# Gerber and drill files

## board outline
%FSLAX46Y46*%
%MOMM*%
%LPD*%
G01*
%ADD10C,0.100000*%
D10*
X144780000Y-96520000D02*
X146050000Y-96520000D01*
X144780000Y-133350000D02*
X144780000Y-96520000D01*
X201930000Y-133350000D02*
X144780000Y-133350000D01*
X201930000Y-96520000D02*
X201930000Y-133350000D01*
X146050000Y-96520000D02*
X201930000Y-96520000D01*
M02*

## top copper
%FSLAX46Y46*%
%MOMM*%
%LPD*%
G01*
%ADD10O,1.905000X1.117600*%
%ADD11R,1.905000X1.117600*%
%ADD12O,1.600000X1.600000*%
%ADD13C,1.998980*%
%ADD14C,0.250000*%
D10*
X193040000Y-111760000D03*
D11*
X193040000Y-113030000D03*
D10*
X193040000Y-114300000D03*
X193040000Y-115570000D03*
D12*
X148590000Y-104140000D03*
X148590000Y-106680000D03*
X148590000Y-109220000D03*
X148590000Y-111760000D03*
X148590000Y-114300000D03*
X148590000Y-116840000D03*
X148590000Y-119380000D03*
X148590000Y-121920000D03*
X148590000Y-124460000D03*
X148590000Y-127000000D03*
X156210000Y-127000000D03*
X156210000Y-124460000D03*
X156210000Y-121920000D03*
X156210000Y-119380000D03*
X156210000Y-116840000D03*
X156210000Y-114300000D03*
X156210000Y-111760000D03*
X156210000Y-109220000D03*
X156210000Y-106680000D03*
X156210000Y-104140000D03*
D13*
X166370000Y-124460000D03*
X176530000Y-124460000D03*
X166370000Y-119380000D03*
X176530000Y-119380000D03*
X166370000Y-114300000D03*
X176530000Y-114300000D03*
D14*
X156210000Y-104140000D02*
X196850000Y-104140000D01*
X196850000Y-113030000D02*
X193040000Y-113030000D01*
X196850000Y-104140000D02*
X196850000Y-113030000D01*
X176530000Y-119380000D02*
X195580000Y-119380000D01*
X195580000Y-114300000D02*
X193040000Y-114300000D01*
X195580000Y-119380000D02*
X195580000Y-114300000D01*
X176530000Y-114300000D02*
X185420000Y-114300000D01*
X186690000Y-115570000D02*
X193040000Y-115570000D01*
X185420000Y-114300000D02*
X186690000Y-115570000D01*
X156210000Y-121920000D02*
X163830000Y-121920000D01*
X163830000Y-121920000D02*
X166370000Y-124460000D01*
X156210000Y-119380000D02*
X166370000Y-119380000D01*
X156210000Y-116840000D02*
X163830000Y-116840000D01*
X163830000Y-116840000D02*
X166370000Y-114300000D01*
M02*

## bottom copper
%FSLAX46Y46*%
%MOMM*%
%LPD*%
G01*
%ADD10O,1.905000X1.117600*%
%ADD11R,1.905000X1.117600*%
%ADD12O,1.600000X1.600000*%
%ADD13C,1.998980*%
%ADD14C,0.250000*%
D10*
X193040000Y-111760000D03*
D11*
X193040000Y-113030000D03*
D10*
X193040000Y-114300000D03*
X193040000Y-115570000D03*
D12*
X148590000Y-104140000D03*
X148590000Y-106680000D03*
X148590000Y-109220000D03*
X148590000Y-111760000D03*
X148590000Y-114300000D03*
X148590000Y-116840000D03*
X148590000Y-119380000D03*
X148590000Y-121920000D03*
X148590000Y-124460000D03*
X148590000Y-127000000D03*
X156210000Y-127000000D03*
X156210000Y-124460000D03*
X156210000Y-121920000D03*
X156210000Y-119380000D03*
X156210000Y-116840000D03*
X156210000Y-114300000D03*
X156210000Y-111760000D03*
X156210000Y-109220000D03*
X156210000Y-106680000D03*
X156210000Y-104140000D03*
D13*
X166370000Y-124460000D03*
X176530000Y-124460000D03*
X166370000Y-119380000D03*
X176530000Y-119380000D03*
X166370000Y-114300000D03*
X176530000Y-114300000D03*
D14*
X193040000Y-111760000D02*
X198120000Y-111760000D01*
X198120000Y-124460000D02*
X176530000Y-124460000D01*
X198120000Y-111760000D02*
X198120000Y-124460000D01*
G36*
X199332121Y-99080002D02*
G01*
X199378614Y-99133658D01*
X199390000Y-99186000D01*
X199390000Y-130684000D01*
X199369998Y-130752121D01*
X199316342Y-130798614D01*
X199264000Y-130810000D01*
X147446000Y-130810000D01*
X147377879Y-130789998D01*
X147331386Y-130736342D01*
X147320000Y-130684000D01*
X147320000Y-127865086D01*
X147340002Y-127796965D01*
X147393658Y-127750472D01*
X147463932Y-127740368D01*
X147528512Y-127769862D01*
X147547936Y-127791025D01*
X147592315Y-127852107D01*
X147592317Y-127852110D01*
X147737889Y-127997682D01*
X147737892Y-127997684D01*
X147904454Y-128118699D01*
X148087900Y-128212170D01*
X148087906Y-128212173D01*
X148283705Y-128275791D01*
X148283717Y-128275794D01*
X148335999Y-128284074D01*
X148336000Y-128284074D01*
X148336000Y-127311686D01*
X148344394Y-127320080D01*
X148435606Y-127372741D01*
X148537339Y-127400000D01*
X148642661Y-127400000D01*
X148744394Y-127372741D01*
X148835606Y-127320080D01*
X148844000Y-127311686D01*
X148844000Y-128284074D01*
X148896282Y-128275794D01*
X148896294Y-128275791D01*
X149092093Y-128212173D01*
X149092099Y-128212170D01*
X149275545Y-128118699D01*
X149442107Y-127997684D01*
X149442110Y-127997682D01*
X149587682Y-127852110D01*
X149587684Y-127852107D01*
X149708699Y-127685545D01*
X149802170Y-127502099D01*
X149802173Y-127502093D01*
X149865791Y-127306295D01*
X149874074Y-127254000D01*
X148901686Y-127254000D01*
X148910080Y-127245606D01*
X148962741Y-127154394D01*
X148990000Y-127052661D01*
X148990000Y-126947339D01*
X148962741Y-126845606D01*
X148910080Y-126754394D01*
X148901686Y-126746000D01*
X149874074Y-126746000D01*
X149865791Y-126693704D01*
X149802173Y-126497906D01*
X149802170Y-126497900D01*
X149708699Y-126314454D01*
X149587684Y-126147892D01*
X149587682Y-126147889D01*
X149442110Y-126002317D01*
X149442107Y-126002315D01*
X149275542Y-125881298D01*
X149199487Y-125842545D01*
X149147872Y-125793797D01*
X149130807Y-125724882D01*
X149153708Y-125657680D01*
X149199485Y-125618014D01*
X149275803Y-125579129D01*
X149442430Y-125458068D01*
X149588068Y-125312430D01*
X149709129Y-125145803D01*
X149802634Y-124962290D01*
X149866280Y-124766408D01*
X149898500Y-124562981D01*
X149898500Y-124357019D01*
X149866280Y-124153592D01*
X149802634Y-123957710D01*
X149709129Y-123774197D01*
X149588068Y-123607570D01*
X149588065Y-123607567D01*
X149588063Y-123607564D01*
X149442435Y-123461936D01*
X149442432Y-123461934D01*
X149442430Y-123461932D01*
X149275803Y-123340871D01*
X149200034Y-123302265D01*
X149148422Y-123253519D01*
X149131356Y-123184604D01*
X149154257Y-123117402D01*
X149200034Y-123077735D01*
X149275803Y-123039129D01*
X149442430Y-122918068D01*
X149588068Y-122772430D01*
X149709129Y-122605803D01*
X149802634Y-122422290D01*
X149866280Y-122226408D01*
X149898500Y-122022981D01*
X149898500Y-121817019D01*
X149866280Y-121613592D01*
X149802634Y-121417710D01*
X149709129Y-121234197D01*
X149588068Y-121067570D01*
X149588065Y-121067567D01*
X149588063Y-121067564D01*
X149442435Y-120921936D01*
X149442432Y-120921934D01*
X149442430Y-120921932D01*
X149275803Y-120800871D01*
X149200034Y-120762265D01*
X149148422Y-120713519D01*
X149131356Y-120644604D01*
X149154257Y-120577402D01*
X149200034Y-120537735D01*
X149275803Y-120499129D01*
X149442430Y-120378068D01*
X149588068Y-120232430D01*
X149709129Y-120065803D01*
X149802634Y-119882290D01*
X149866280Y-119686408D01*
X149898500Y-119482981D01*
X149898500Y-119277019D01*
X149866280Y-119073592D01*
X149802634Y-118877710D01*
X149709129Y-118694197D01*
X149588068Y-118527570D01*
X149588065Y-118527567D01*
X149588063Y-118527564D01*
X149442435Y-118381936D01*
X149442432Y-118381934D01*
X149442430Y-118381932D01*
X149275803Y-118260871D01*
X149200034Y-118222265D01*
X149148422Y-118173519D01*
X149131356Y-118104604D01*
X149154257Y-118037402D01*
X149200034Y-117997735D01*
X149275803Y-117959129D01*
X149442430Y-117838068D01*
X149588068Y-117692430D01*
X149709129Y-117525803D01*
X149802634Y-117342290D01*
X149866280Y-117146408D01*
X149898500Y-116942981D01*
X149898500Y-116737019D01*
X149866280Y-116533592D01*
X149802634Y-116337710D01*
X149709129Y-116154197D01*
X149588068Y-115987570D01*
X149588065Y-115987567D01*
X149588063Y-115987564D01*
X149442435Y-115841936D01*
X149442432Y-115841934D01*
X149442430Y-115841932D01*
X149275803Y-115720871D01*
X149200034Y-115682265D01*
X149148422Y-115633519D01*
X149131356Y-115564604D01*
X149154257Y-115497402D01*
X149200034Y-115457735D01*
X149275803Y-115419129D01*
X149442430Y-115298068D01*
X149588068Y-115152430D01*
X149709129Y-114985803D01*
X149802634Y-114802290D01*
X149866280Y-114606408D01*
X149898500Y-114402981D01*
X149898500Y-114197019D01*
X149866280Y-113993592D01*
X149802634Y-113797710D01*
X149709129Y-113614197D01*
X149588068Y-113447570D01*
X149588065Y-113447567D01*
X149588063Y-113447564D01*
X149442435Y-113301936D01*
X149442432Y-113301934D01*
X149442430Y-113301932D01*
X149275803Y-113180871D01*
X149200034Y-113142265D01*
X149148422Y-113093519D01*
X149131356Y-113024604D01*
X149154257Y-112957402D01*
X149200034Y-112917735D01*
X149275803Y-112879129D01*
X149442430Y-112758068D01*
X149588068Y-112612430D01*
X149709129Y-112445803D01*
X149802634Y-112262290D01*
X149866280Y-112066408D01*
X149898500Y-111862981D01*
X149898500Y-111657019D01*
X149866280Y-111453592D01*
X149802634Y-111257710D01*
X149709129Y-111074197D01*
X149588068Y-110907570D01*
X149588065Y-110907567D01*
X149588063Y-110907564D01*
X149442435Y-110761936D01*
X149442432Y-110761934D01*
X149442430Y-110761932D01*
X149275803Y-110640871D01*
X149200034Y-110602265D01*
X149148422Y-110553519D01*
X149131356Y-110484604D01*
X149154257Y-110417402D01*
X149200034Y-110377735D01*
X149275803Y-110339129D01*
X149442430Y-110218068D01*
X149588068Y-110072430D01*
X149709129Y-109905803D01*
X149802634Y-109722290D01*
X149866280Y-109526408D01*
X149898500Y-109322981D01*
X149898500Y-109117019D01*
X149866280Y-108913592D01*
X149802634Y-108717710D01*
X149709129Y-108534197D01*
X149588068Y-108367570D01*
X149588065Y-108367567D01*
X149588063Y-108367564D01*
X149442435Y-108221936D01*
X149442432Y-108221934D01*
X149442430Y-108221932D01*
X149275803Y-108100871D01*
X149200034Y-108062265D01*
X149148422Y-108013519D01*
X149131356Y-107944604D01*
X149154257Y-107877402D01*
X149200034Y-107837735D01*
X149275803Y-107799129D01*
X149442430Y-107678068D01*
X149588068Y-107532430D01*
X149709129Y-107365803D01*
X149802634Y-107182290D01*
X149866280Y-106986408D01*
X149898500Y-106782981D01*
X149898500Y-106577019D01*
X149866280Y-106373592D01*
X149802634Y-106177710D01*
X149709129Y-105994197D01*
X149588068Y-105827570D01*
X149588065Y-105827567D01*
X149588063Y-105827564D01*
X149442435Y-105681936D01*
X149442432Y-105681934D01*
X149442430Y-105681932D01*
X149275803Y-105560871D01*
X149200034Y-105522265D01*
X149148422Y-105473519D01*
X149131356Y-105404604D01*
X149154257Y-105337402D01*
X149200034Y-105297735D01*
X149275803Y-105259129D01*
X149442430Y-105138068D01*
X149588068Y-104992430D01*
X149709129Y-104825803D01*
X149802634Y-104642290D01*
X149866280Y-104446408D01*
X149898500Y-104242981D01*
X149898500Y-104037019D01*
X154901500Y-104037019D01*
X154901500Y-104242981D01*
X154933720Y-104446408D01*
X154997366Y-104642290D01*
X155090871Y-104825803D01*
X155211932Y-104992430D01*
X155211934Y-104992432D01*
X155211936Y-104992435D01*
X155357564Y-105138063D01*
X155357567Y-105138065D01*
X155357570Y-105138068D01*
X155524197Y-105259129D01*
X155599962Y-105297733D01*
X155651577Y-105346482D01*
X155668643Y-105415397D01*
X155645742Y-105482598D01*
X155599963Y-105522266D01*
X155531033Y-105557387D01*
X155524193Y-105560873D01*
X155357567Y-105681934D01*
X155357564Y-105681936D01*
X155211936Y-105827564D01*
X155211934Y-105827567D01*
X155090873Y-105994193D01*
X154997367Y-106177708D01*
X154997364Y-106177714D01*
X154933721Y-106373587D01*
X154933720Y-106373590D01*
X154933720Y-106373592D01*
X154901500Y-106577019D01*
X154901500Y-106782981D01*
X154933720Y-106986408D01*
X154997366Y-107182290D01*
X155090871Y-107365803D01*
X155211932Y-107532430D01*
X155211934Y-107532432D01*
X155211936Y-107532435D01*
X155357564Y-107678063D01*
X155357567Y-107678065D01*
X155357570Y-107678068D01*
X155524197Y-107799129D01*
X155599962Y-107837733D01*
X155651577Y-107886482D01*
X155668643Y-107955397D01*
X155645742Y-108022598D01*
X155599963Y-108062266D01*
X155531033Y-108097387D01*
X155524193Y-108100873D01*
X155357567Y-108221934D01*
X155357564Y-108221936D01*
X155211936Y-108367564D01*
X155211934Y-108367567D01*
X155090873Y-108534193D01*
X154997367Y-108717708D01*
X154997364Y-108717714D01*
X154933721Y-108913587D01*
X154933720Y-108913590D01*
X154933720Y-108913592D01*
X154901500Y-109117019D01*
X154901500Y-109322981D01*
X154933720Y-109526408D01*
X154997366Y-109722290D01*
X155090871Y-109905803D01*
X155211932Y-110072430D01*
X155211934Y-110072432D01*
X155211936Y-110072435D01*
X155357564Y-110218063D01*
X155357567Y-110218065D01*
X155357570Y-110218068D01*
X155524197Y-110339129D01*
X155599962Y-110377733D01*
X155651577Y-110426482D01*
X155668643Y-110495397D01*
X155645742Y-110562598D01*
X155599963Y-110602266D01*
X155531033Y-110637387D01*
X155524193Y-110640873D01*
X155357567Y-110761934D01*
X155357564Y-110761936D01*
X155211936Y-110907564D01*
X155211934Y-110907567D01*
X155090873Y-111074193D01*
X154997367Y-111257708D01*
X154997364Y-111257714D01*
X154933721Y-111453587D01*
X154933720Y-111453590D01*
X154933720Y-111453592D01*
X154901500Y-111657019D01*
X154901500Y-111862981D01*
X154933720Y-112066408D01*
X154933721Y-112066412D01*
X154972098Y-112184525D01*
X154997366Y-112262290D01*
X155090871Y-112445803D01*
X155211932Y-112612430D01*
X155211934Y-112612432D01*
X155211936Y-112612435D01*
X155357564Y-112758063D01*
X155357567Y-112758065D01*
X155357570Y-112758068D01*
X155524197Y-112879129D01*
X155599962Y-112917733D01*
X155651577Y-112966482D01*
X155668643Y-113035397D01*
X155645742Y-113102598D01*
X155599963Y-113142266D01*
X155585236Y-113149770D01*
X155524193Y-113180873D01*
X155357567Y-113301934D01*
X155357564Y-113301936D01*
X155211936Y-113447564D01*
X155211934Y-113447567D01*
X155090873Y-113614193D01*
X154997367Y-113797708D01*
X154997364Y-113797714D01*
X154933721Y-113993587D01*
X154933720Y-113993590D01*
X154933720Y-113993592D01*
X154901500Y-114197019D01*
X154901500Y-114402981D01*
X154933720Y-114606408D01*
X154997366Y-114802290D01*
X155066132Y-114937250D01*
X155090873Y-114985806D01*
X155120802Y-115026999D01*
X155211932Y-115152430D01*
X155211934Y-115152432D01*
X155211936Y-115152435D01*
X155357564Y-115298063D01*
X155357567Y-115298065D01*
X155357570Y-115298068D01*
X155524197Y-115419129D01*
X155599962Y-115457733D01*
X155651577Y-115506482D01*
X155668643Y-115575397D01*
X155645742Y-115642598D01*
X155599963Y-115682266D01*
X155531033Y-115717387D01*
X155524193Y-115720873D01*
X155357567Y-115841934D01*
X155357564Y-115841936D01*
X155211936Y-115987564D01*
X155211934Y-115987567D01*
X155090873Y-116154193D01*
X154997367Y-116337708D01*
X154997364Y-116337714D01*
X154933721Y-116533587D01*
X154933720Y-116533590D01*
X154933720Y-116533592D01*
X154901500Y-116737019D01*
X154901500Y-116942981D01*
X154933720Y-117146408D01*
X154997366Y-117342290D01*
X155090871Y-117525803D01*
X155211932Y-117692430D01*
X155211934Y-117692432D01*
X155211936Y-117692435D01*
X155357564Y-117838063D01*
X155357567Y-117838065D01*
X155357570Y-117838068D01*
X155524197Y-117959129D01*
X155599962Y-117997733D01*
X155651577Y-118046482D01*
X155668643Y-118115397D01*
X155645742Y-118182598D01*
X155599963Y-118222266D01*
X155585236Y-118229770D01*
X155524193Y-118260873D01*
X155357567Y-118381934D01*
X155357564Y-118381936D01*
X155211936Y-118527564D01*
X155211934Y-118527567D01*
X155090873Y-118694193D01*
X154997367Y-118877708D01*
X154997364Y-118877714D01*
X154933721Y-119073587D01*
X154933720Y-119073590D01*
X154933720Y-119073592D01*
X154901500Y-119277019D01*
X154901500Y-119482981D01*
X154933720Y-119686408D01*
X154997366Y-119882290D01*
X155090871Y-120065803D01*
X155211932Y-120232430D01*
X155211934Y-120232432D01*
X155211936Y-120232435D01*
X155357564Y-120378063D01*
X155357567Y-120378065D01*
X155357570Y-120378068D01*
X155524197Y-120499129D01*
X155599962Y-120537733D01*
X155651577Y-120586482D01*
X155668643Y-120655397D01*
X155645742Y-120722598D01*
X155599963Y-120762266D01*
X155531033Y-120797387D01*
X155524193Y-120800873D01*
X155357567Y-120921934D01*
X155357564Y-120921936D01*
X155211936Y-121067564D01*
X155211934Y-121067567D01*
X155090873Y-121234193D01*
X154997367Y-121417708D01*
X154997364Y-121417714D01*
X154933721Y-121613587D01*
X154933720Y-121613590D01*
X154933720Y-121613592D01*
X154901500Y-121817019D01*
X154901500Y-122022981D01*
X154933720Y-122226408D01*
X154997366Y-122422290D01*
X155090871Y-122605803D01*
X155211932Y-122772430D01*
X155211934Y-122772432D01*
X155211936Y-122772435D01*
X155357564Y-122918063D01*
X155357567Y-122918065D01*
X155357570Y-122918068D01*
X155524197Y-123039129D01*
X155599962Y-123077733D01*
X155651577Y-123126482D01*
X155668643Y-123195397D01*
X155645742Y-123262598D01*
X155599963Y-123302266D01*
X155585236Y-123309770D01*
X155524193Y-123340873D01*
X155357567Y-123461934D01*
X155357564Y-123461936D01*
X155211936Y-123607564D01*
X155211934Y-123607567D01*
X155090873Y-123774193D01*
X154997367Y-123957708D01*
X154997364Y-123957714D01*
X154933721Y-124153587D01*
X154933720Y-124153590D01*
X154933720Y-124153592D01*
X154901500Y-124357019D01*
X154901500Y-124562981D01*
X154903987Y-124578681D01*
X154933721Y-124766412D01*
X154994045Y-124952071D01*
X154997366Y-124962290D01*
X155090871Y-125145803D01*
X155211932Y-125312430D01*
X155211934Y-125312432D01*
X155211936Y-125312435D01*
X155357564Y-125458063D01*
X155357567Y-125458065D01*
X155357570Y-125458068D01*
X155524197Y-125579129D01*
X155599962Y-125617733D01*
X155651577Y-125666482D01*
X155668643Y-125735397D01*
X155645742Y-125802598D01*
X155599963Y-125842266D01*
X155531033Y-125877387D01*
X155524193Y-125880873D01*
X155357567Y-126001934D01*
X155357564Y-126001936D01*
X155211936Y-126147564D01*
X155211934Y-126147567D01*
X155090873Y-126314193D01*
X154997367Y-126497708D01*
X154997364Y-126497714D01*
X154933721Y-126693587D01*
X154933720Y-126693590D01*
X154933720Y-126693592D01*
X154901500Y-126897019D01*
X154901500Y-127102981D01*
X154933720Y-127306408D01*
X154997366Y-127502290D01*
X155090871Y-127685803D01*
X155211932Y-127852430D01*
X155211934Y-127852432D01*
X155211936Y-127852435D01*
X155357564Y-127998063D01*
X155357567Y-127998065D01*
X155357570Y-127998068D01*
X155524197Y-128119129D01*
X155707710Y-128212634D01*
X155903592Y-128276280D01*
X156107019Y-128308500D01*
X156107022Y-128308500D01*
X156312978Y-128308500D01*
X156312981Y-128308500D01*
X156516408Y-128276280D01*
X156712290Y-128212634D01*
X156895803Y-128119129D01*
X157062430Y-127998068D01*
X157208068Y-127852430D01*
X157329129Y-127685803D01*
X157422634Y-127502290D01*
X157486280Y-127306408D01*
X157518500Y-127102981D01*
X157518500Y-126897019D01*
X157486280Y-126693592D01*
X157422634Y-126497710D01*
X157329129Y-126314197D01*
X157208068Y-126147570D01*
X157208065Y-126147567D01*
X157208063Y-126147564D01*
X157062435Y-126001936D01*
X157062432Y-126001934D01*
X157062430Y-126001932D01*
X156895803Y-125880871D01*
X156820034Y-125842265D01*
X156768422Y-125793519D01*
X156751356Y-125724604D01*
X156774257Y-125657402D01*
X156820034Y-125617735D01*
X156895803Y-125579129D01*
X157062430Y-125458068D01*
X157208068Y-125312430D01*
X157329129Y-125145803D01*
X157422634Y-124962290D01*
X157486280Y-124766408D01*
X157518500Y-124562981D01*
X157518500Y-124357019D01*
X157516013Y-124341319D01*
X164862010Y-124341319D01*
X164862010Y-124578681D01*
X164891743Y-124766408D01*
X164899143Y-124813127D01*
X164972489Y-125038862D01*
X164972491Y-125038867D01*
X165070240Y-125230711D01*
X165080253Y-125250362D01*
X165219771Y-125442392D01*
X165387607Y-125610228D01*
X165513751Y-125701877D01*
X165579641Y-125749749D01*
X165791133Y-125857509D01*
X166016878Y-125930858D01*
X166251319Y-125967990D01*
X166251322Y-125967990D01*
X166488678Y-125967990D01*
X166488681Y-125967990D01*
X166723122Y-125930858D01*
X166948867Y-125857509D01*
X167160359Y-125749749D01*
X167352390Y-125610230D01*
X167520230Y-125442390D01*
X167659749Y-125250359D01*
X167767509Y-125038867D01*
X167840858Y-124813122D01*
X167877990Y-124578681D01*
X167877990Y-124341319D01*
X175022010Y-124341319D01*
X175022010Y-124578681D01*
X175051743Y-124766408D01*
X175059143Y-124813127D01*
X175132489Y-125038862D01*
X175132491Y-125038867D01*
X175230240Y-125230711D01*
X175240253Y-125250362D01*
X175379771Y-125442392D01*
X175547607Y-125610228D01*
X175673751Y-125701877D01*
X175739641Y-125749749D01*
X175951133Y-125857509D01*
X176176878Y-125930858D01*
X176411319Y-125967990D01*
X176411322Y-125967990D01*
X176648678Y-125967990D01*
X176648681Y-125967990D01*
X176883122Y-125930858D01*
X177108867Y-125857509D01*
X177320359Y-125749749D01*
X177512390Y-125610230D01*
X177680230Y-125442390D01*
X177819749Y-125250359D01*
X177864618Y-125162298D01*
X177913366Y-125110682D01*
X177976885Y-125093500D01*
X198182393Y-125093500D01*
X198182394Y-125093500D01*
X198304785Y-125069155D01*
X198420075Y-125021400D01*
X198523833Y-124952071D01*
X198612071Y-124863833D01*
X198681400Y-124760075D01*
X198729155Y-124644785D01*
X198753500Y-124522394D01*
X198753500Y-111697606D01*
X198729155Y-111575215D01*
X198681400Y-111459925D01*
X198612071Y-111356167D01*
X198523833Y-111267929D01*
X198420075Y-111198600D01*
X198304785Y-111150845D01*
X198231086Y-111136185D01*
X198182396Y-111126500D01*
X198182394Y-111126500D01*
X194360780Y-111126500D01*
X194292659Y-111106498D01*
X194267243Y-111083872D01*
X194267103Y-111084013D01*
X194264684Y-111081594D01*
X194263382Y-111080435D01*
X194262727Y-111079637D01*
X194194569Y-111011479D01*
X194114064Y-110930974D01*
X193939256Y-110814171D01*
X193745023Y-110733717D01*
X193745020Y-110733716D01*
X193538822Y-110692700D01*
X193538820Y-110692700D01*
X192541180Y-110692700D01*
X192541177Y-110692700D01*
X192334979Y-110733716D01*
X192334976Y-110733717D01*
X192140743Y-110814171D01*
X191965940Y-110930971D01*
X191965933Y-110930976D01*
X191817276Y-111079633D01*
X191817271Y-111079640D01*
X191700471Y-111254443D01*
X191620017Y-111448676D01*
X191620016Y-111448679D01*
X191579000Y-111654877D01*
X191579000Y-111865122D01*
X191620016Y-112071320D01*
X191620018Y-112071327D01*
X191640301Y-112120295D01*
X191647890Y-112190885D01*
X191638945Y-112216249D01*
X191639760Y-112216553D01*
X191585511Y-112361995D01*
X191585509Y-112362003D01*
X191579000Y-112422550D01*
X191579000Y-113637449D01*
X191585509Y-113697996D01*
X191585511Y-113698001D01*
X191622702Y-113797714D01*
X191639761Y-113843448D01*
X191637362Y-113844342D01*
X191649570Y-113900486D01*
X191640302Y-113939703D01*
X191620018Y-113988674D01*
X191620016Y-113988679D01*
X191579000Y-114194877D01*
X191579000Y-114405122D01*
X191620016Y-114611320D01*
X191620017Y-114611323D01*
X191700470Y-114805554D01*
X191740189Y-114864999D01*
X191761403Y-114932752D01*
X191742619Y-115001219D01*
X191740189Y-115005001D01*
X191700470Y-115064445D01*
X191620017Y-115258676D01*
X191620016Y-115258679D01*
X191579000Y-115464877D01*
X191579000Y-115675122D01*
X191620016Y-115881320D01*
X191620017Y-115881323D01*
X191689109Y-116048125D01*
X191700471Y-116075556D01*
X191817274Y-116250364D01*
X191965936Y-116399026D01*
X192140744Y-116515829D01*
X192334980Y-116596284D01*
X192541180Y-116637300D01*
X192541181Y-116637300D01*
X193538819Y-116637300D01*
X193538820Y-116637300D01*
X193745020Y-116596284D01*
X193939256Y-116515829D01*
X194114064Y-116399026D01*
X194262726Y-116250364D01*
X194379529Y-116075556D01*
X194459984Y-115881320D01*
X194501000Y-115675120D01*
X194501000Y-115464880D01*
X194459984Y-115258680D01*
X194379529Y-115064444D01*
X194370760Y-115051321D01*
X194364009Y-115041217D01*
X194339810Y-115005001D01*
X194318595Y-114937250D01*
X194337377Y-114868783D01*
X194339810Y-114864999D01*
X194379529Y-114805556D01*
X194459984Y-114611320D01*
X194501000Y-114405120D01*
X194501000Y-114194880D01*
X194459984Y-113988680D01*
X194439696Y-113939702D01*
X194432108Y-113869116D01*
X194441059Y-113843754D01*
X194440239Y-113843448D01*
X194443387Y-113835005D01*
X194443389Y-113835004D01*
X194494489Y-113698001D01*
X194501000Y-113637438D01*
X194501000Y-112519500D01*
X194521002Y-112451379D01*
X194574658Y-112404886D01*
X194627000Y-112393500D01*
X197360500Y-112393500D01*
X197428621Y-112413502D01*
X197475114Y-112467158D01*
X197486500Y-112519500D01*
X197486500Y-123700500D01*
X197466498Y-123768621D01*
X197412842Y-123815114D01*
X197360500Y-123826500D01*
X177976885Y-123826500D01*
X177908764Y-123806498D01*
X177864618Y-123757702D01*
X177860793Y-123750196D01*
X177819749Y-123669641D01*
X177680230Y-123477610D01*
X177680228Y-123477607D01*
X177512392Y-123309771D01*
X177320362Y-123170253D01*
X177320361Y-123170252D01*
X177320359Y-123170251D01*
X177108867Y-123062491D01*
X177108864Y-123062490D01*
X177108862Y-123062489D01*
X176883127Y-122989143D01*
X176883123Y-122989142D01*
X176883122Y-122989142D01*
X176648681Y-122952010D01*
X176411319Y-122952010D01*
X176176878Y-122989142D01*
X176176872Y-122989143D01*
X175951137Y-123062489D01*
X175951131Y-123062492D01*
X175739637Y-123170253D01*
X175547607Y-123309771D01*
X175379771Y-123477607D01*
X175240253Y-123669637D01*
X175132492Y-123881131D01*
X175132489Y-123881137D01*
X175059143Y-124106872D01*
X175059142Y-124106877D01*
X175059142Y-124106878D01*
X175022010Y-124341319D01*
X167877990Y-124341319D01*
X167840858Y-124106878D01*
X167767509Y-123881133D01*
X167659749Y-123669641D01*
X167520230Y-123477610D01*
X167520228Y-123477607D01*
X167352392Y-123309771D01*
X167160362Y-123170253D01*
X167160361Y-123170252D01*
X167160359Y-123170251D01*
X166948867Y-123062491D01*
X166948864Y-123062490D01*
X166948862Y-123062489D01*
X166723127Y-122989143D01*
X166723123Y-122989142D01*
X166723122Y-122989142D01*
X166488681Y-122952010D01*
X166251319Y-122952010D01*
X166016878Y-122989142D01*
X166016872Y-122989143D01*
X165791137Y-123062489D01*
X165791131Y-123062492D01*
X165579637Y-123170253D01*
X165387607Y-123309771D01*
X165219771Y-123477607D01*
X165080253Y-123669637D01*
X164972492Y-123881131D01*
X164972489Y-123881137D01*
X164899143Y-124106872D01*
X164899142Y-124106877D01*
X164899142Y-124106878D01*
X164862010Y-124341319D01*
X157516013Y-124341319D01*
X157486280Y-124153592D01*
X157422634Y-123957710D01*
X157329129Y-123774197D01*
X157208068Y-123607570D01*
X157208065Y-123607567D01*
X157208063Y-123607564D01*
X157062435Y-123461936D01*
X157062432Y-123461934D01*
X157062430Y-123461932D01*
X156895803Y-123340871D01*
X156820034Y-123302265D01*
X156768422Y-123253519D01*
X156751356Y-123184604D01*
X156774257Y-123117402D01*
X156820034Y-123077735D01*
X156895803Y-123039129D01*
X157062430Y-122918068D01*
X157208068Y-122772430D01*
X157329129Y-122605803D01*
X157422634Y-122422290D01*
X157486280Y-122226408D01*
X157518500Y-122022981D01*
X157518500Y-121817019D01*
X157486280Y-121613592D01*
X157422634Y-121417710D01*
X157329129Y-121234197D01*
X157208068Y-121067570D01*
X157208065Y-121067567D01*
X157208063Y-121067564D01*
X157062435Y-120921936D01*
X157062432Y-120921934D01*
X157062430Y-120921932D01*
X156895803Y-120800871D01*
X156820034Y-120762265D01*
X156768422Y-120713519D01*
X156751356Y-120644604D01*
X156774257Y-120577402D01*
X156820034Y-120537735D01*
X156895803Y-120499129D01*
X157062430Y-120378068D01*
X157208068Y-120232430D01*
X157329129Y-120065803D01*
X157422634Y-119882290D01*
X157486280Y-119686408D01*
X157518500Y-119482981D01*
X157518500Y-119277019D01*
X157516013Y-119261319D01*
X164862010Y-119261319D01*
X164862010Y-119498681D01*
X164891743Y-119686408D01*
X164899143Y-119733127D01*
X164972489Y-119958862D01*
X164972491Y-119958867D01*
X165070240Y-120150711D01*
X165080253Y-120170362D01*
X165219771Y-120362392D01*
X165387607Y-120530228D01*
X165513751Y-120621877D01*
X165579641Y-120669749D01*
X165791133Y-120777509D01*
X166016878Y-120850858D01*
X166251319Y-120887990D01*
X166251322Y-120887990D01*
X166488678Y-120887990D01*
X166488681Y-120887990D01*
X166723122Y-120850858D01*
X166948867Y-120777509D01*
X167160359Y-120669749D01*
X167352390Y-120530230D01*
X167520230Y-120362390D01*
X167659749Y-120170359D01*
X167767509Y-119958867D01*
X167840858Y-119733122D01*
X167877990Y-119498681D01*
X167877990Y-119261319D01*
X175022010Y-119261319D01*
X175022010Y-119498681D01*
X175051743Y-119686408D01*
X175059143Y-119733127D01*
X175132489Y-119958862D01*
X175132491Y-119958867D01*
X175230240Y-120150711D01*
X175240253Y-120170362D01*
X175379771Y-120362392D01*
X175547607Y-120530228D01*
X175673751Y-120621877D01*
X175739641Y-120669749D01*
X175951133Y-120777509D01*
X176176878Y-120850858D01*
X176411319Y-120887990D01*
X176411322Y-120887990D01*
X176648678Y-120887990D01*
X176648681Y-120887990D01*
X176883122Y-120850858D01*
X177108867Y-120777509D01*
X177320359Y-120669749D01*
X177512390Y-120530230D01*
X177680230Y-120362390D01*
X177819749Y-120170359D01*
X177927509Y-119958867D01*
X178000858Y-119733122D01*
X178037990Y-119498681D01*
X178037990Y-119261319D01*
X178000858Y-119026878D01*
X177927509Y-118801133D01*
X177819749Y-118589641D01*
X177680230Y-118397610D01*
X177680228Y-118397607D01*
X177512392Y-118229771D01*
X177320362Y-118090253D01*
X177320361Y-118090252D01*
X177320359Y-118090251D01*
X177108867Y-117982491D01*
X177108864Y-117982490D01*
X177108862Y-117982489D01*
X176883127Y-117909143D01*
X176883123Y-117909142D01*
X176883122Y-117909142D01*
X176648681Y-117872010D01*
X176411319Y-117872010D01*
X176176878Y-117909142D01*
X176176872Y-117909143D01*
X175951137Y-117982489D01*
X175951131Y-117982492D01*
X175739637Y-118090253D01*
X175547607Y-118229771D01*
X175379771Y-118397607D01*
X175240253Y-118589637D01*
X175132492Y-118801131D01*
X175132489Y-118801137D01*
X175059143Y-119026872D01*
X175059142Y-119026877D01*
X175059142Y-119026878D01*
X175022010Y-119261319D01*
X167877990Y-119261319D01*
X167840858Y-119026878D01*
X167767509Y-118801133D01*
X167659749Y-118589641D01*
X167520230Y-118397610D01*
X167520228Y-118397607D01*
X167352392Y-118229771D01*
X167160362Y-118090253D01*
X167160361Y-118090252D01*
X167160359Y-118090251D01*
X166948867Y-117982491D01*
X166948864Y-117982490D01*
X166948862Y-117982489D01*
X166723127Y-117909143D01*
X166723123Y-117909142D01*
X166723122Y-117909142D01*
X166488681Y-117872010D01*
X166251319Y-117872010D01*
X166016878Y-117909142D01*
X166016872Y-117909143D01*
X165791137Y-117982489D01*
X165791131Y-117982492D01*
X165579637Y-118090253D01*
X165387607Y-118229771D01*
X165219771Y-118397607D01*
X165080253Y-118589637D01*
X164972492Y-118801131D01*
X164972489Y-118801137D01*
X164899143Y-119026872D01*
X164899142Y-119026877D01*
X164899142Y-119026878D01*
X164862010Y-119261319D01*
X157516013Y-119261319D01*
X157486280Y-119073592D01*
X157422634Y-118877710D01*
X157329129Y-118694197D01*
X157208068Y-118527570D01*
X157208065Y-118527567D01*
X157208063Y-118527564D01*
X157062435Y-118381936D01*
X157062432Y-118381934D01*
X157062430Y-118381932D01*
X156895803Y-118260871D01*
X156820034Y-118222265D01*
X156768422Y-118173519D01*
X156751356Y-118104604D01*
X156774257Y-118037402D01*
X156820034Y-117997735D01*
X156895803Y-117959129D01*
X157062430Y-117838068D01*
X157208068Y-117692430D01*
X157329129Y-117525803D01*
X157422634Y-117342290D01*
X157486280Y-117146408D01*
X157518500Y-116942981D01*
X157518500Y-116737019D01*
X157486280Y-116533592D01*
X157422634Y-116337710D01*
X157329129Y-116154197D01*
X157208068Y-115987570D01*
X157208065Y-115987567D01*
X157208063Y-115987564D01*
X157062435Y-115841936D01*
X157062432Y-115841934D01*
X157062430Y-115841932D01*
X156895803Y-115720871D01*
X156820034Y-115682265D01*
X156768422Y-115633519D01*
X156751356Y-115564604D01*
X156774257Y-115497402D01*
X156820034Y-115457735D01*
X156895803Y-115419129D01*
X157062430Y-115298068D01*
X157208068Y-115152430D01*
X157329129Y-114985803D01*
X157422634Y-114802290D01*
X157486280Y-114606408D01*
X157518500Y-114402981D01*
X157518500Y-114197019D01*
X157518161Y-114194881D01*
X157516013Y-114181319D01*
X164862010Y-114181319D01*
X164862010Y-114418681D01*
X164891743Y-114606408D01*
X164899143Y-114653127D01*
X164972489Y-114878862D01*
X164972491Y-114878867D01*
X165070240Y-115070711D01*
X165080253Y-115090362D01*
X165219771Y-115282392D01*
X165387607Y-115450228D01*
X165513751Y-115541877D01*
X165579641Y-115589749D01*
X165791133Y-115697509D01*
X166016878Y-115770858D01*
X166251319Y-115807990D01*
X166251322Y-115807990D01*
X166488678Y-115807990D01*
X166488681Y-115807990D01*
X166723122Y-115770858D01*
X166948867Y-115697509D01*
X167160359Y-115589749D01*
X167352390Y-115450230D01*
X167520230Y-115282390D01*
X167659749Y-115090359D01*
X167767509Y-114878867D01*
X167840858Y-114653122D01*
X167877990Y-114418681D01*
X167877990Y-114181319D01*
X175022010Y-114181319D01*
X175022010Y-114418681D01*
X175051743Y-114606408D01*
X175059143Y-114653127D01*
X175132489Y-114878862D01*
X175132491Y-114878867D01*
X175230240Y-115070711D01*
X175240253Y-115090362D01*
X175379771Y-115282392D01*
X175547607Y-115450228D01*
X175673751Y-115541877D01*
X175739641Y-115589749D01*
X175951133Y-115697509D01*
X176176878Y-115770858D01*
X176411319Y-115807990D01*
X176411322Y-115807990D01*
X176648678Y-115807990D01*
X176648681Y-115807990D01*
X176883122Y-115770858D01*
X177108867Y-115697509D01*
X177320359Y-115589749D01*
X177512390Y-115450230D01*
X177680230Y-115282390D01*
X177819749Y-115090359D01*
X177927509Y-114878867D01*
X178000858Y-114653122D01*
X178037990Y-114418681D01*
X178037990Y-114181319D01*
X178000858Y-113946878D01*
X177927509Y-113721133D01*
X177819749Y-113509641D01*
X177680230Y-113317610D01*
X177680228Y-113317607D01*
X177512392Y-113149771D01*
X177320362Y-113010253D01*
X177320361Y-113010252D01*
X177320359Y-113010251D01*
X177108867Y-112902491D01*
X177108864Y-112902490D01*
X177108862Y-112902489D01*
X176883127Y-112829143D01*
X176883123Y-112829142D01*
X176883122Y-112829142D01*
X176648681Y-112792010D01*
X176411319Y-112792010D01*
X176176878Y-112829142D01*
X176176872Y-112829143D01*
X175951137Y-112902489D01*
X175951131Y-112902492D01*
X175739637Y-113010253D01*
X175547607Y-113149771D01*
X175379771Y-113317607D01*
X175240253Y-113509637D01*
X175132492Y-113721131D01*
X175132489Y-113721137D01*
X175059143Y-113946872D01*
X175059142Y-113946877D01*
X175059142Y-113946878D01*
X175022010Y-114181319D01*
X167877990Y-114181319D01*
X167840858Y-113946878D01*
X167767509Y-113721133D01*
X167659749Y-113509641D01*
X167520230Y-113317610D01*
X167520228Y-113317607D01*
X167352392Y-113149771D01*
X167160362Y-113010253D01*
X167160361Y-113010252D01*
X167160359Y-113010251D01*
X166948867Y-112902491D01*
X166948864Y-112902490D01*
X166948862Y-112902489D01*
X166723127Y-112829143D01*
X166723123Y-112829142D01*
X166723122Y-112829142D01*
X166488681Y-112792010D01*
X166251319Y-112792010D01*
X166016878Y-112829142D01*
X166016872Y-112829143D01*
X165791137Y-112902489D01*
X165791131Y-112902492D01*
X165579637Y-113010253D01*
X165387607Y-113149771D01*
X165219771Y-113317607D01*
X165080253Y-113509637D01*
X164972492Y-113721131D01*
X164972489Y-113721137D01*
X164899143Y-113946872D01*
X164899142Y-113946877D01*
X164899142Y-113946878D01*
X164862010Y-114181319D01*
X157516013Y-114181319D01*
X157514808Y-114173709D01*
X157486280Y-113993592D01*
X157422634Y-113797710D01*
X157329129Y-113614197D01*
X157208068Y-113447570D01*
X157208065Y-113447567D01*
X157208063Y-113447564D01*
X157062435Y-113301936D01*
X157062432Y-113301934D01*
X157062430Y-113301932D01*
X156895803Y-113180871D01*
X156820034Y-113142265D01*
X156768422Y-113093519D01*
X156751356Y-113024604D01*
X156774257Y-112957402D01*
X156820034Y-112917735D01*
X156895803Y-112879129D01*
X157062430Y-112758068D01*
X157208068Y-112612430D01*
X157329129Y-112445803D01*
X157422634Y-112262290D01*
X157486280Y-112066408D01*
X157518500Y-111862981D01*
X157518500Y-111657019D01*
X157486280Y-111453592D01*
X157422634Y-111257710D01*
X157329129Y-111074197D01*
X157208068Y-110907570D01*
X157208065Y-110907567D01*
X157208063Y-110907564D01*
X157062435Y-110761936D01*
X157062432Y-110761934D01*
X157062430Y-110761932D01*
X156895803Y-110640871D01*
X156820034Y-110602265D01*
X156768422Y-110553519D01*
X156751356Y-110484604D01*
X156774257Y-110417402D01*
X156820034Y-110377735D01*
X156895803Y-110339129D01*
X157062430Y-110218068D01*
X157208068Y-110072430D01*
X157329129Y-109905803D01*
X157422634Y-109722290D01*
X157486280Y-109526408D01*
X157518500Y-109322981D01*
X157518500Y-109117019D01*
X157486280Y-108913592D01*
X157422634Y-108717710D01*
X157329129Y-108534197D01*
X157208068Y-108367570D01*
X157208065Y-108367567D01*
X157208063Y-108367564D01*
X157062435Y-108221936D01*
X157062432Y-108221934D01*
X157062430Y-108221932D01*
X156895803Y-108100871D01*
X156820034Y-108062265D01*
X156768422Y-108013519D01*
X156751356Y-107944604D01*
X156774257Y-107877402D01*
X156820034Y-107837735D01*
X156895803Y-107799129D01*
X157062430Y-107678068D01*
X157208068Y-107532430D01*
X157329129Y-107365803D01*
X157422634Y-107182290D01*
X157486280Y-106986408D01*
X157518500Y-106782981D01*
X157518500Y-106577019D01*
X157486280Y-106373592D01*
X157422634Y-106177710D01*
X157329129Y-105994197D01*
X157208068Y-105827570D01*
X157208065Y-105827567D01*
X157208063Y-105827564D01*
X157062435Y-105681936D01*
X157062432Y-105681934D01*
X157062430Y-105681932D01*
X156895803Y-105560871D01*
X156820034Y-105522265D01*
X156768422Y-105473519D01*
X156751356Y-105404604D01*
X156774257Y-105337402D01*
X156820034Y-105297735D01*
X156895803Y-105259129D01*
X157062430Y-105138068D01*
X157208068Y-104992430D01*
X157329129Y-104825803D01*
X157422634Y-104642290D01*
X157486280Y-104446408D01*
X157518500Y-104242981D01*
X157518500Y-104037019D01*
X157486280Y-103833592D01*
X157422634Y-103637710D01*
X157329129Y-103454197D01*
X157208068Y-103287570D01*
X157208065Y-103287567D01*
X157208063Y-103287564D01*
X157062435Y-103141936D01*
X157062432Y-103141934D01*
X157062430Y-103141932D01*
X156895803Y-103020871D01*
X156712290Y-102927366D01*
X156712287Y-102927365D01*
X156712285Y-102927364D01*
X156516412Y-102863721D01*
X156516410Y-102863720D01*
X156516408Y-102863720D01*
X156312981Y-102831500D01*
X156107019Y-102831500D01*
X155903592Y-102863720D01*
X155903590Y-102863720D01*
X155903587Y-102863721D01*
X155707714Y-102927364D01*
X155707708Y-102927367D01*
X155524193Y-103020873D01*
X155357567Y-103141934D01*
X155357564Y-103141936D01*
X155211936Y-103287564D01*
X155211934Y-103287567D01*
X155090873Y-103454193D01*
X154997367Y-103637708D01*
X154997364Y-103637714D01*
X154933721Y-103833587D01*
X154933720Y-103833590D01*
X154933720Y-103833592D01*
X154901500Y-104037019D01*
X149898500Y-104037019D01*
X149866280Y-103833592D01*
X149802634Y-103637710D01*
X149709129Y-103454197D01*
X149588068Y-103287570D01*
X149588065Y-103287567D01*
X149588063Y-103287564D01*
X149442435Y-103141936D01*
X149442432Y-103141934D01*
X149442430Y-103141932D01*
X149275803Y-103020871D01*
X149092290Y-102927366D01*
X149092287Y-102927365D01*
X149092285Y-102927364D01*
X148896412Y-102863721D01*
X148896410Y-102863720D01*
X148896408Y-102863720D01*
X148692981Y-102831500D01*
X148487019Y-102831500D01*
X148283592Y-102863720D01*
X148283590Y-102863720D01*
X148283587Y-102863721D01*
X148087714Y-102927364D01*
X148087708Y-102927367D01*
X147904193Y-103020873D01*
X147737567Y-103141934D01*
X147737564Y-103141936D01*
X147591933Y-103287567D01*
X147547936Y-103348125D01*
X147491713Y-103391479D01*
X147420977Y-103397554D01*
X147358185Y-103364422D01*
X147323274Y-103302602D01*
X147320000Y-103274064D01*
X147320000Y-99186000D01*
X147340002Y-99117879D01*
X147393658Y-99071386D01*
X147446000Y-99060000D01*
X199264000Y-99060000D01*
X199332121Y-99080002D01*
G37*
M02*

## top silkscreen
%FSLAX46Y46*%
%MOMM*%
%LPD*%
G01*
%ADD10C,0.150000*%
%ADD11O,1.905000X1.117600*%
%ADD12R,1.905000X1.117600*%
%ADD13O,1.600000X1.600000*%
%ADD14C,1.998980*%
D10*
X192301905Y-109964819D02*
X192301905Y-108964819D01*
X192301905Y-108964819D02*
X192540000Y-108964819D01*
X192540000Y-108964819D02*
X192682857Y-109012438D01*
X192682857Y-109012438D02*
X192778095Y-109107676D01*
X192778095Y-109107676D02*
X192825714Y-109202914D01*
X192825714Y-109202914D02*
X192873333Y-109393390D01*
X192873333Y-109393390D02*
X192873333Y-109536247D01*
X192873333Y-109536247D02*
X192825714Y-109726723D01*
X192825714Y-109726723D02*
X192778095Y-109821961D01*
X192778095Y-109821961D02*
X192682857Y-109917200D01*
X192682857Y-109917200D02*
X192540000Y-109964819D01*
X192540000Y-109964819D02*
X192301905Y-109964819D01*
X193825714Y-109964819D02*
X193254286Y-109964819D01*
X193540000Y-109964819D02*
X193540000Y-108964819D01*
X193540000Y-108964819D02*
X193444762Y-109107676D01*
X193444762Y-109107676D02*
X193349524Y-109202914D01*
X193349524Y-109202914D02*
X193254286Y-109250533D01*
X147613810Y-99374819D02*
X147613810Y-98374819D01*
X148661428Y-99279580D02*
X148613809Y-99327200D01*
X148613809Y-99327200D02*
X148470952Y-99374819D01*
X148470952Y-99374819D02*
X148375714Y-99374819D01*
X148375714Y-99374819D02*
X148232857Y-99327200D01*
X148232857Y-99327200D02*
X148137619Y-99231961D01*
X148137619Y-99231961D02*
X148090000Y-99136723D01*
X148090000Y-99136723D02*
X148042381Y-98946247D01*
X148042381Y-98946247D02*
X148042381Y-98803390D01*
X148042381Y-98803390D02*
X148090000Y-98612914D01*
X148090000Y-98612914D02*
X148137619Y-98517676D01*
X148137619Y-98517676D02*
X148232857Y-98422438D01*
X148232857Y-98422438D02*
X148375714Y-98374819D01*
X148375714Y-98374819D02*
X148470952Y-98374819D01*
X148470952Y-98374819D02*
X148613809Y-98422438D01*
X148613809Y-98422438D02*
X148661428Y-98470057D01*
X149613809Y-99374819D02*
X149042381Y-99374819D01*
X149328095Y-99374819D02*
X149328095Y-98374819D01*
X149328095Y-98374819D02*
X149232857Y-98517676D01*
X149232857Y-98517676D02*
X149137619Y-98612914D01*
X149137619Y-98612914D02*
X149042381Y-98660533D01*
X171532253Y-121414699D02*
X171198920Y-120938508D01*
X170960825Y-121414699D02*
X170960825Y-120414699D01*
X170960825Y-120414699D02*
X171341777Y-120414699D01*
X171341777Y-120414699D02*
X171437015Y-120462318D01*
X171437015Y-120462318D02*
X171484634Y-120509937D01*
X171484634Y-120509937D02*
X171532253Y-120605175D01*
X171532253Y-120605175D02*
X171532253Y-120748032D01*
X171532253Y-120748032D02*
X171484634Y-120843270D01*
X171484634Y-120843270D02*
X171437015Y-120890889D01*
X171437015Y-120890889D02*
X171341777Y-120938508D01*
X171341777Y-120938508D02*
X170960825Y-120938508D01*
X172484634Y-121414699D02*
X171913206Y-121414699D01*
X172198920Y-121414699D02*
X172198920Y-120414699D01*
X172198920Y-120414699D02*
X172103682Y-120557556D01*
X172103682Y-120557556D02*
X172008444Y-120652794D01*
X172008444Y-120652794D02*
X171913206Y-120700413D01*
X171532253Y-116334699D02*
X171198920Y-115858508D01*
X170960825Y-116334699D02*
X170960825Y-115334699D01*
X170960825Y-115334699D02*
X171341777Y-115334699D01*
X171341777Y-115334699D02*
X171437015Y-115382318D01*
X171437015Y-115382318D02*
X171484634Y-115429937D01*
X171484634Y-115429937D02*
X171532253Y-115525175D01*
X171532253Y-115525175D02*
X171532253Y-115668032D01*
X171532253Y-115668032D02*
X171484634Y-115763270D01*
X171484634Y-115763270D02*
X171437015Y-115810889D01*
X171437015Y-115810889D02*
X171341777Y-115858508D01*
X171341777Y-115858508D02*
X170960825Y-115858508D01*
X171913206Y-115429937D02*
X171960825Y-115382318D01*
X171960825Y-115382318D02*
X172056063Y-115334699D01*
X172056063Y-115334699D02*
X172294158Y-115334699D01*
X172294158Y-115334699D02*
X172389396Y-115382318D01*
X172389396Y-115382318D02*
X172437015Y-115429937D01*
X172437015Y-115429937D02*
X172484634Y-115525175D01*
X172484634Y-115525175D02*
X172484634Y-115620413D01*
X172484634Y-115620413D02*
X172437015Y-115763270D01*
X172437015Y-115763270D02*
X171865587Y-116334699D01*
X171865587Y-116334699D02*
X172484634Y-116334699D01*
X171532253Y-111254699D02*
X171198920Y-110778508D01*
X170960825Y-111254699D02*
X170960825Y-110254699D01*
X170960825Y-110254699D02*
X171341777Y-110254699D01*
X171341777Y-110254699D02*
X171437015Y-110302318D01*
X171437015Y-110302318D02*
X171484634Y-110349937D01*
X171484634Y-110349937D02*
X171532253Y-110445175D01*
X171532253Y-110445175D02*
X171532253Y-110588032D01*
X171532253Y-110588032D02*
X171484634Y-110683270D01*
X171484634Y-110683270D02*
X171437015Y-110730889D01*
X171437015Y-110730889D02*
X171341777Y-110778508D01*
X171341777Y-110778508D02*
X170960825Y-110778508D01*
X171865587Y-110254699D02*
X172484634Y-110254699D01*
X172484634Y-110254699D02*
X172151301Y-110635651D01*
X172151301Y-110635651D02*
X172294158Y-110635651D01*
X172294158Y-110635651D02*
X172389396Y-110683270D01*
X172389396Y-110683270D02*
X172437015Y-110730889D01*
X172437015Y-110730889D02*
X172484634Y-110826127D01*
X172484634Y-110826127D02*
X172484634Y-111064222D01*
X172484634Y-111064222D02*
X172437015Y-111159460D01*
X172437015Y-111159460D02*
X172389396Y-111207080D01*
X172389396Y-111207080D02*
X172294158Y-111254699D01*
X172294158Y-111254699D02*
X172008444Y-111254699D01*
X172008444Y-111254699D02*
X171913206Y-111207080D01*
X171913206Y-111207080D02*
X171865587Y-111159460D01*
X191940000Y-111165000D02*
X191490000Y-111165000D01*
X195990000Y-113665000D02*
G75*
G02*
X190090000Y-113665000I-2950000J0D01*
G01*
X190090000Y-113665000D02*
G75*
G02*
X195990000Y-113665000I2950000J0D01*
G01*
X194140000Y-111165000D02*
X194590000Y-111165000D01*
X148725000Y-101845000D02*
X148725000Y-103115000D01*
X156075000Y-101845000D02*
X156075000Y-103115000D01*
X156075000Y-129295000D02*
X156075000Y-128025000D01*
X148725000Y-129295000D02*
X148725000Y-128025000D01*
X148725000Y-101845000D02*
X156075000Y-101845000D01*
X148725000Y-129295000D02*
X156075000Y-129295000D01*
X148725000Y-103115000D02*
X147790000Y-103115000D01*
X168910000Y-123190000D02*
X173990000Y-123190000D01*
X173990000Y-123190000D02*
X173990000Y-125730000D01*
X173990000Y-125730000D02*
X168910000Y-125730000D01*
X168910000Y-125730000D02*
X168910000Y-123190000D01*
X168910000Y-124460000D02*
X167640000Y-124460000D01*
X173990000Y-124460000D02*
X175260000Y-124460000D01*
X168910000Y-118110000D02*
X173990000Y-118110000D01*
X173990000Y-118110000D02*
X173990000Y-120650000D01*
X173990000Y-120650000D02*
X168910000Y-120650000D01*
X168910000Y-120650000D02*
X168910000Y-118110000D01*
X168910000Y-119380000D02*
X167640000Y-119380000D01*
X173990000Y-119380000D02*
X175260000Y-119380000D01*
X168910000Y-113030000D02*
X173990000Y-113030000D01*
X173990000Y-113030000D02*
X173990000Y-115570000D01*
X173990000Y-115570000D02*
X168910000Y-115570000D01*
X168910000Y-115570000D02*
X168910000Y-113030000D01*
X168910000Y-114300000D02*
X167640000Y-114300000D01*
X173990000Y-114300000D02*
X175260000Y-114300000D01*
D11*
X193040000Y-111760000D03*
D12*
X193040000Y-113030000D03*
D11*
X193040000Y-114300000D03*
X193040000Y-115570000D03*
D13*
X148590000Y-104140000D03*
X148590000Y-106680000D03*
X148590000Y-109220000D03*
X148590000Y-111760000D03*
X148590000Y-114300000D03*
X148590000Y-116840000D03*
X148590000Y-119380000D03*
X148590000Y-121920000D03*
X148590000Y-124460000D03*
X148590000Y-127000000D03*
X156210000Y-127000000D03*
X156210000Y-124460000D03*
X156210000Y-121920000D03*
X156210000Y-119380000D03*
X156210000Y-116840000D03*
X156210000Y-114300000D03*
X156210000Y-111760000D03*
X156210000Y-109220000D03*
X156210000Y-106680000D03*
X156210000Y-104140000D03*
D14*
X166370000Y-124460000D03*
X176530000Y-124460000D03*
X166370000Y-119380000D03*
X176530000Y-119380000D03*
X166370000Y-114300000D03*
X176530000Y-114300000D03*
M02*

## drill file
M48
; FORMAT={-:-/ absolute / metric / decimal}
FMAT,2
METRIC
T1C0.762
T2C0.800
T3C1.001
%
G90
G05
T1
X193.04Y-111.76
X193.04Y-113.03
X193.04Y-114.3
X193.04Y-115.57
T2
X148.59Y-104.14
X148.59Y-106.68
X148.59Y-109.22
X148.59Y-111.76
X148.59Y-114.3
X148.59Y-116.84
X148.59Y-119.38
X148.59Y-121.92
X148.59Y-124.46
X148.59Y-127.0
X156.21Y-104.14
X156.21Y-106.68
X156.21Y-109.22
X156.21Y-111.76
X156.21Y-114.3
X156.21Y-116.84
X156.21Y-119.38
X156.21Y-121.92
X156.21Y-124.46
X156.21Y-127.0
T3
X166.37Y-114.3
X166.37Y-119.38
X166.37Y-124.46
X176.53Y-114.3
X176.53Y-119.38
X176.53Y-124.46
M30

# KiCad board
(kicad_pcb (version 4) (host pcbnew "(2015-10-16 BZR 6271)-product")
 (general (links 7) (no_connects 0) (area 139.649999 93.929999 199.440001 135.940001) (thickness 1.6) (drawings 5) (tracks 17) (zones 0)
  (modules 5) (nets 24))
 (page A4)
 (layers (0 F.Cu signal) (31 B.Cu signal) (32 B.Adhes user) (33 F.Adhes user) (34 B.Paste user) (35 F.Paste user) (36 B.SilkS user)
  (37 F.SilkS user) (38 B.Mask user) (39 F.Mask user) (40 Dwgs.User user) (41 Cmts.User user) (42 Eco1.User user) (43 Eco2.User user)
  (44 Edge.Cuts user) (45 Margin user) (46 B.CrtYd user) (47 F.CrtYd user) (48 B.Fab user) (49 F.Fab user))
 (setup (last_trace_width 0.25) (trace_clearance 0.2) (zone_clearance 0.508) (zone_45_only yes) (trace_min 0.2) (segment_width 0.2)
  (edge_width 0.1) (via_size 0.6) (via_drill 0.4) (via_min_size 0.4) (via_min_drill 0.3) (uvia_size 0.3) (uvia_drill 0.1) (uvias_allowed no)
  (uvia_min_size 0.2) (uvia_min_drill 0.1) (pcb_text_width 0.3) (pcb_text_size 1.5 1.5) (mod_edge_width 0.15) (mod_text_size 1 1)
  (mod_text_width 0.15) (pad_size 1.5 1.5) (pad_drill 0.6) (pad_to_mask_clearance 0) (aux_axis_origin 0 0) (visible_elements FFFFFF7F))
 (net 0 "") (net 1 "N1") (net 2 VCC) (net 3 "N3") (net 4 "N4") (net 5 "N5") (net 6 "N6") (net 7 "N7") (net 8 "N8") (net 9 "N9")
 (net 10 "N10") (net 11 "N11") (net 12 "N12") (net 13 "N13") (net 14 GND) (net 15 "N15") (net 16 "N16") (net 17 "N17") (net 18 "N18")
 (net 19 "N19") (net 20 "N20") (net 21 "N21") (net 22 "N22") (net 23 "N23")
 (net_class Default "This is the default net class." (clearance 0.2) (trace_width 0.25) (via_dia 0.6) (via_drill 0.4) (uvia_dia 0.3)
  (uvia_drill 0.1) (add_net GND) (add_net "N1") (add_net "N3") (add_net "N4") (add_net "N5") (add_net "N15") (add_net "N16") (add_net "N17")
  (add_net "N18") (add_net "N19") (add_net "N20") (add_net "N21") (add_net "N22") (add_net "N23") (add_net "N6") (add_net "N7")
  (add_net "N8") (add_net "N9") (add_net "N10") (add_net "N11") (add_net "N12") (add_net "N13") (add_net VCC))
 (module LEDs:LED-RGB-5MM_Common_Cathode (layer F.Cu) (at 193.04 111.76)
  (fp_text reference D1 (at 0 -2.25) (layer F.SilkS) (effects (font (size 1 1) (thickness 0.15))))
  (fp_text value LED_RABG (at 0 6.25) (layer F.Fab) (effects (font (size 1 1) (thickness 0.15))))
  (fp_line (start -1.1 -0.595) (end -1.55 -0.595) (layer F.SilkS) (width 0.15))
  (fp_circle (center 0 1.905) (end 2.95 1.905) (layer F.SilkS) (width 0.15))
  (fp_line (start 1.1 -0.595) (end 1.55 -0.595) (layer F.SilkS) (width 0.15))
  (pad 1 thru_hole oval (at 0 0) (size 1.905 1.1176) (drill 0.762) (layers *.Cu *.Mask F.SilkS) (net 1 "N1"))
  (pad 2 thru_hole rect (at 0 1.27) (size 1.905 1.1176) (drill 0.762) (layers *.Cu *.Mask F.SilkS) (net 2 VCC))
  (pad 3 thru_hole oval (at 0 2.54) (size 1.905 1.1176) (drill 0.762) (layers *.Cu *.Mask F.SilkS) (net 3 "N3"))
  (pad 4 thru_hole oval (at 0 3.81) (size 1.905 1.1176) (drill 0.762) (layers *.Cu *.Mask F.SilkS) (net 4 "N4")))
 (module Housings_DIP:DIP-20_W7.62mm (layer F.Cu) (at 148.59 104.14)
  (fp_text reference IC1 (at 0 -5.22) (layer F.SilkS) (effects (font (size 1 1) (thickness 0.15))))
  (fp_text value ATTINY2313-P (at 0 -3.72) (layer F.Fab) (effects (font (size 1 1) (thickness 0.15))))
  (fp_line (start 0.135 -2.295) (end 0.135 -1.025) (layer F.SilkS) (width 0.15))
  (fp_line (start 7.485 -2.295) (end 7.485 -1.025) (layer F.SilkS) (width 0.15))
  (fp_line (start 7.485 25.155) (end 7.485 23.885) (layer F.SilkS) (width 0.15))
  (fp_line (start 0.135 25.155) (end 0.135 23.885) (layer F.SilkS) (width 0.15))
  (fp_line (start 0.135 -2.295) (end 7.485 -2.295) (layer F.SilkS) (width 0.15))
  (fp_line (start 0.135 25.155) (end 7.485 25.155) (layer F.SilkS) (width 0.15))
  (fp_line (start 0.135 -1.025) (end -0.8 -1.025) (layer F.SilkS) (width 0.15))
  (pad 1 thru_hole oval (at 0 0) (size 1.6 1.6) (drill 0.8) (layers *.Cu *.Mask F.SilkS) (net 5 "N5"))
  (pad 2 thru_hole oval (at 0 2.54) (size 1.6 1.6) (drill 0.8) (layers *.Cu *.Mask F.SilkS) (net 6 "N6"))
  (pad 3 thru_hole oval (at 0 5.08) (size 1.6 1.6) (drill 0.8) (layers *.Cu *.Mask F.SilkS) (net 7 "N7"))
  (pad 4 thru_hole oval (at 0 7.62) (size 1.6 1.6) (drill 0.8) (layers *.Cu *.Mask F.SilkS) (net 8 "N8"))
  (pad 5 thru_hole oval (at 0 10.16) (size 1.6 1.6) (drill 0.8) (layers *.Cu *.Mask F.SilkS) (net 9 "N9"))
  (pad 6 thru_hole oval (at 0 12.7) (size 1.6 1.6) (drill 0.8) (layers *.Cu *.Mask F.SilkS) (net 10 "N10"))
  (pad 7 thru_hole oval (at 0 15.24) (size 1.6 1.6) (drill 0.8) (layers *.Cu *.Mask F.SilkS) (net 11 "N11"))
  (pad 8 thru_hole oval (at 0 17.78) (size 1.6 1.6) (drill 0.8) (layers *.Cu *.Mask F.SilkS) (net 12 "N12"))
  (pad 9 thru_hole oval (at 0 20.32) (size 1.6 1.6) (drill 0.8) (layers *.Cu *.Mask F.SilkS) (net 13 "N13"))
  (pad 10 thru_hole oval (at 0 22.86) (size 1.6 1.6) (drill 0.8) (layers *.Cu *.Mask F.SilkS) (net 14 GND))
  (pad 11 thru_hole oval (at 7.62 22.86) (size 1.6 1.6) (drill 0.8) (layers *.Cu *.Mask F.SilkS) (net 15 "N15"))
  (pad 12 thru_hole oval (at 7.62 20.32) (size 1.6 1.6) (drill 0.8) (layers *.Cu *.Mask F.SilkS) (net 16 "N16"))
  (pad 13 thru_hole oval (at 7.62 17.78) (size 1.6 1.6) (drill 0.8) (layers *.Cu *.Mask F.SilkS) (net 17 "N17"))
  (pad 14 thru_hole oval (at 7.62 15.24) (size 1.6 1.6) (drill 0.8) (layers *.Cu *.Mask F.SilkS) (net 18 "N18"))
  (pad 15 thru_hole oval (at 7.62 12.7) (size 1.6 1.6) (drill 0.8) (layers *.Cu *.Mask F.SilkS) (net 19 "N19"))
  (pad 16 thru_hole oval (at 7.62 10.16) (size 1.6 1.6) (drill 0.8) (layers *.Cu *.Mask F.SilkS) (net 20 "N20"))
  (pad 17 thru_hole oval (at 7.62 7.62) (size 1.6 1.6) (drill 0.8) (layers *.Cu *.Mask F.SilkS) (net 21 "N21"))
  (pad 18 thru_hole oval (at 7.62 5.08) (size 1.6 1.6) (drill 0.8) (layers *.Cu *.Mask F.SilkS) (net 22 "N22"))
  (pad 19 thru_hole oval (at 7.62 2.54) (size 1.6 1.6) (drill 0.8) (layers *.Cu *.Mask F.SilkS) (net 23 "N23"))
  (pad 20 thru_hole oval (at 7.62 0) (size 1.6 1.6) (drill 0.8) (layers *.Cu *.Mask F.SilkS) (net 2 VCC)))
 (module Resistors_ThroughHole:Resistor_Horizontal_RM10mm (layer F.Cu) (at 171.45 124.46)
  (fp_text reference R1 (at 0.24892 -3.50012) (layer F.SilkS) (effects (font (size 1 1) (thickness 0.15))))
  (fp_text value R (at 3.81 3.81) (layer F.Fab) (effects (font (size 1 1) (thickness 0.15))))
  (fp_line (start -2.54 -1.27) (end 2.54 -1.27) (layer F.SilkS) (width 0.15))
  (fp_line (start 2.54 -1.27) (end 2.54 1.27) (layer F.SilkS) (width 0.15))
  (fp_line (start 2.54 1.27) (end -2.54 1.27) (layer F.SilkS) (width 0.15))
  (fp_line (start -2.54 1.27) (end -2.54 -1.27) (layer F.SilkS) (width 0.15))
  (fp_line (start -2.54 0) (end -3.81 0) (layer F.SilkS) (width 0.15))
  (fp_line (start 2.54 0) (end 3.81 0) (layer F.SilkS) (width 0.15))
  (pad 1 thru_hole circle (at -5.08 0) (size 1.99898 1.99898) (drill 1.00076) (layers *.Cu *.SilkS *.Mask) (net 17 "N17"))
  (pad 2 thru_hole circle (at 5.08 0) (size 1.99898 1.99898) (drill 1.00076) (layers *.Cu *.SilkS *.Mask) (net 1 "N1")))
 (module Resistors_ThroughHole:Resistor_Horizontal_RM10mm (layer F.Cu) (at 171.45 119.38)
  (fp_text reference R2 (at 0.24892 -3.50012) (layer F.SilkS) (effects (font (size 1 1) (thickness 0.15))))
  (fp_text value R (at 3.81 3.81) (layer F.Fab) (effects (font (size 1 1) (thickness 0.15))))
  (fp_line (start -2.54 -1.27) (end 2.54 -1.27) (layer F.SilkS) (width 0.15))
  (fp_line (start 2.54 -1.27) (end 2.54 1.27) (layer F.SilkS) (width 0.15))
  (fp_line (start 2.54 1.27) (end -2.54 1.27) (layer F.SilkS) (width 0.15))
  (fp_line (start -2.54 1.27) (end -2.54 -1.27) (layer F.SilkS) (width 0.15))
  (fp_line (start -2.54 0) (end -3.81 0) (layer F.SilkS) (width 0.15))
  (fp_line (start 2.54 0) (end 3.81 0) (layer F.SilkS) (width 0.15))
  (pad 1 thru_hole circle (at -5.08 0) (size 1.99898 1.99898) (drill 1.00076) (layers *.Cu *.SilkS *.Mask) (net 18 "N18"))
  (pad 2 thru_hole circle (at 5.08 0) (size 1.99898 1.99898) (drill 1.00076) (layers *.Cu *.SilkS *.Mask) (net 3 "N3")))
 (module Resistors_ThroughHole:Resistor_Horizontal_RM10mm (layer F.Cu) (at 171.45 114.3)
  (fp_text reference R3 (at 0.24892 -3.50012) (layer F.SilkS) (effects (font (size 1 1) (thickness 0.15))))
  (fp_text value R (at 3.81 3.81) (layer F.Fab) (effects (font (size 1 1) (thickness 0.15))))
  (fp_line (start -2.54 -1.27) (end 2.54 -1.27) (layer F.SilkS) (width 0.15))
  (fp_line (start 2.54 -1.27) (end 2.54 1.27) (layer F.SilkS) (width 0.15))
  (fp_line (start 2.54 1.27) (end -2.54 1.27) (layer F.SilkS) (width 0.15))
  (fp_line (start -2.54 1.27) (end -2.54 -1.27) (layer F.SilkS) (width 0.15))
  (fp_line (start -2.54 0) (end -3.81 0) (layer F.SilkS) (width 0.15))
  (fp_line (start 2.54 0) (end 3.81 0) (layer F.SilkS) (width 0.15))
  (pad 1 thru_hole circle (at -5.08 0) (size 1.99898 1.99898) (drill 1.00076) (layers *.Cu *.SilkS *.Mask) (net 19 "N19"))
  (pad 2 thru_hole circle (at 5.08 0) (size 1.99898 1.99898) (drill 1.00076) (layers *.Cu *.SilkS *.Mask) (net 4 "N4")))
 (gr_line (start 144.78 96.52) (end 146.05 96.52) (angle 90) (layer Edge.Cuts) (width 0.1))
 (gr_line (start 144.78 133.35) (end 144.78 96.52) (angle 90) (layer Edge.Cuts) (width 0.1))
 (gr_line (start 201.93 133.35) (end 144.78 133.35) (angle 90) (layer Edge.Cuts) (width 0.1))
 (gr_line (start 201.93 96.52) (end 201.93 133.35) (angle 90) (layer Edge.Cuts) (width 0.1))
 (gr_line (start 146.05 96.52) (end 201.93 96.52) (angle 90) (layer Edge.Cuts) (width 0.1))
 (segment (start 193.04 111.76) (end 198.12 111.76) (width 0.25) (layer B.Cu) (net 1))
 (segment (start 198.12 124.46) (end 176.53 124.46) (width 0.25) (layer B.Cu) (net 1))
 (segment (start 198.12 111.76) (end 198.12 124.46) (width 0.25) (layer B.Cu) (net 1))
 (segment (start 156.21 104.14) (end 196.85 104.14) (width 0.25) (layer F.Cu) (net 2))
 (segment (start 196.85 113.03) (end 193.04 113.03) (width 0.25) (layer F.Cu) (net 2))
 (segment (start 196.85 104.14) (end 196.85 113.03) (width 0.25) (layer F.Cu) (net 2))
 (segment (start 176.53 119.38) (end 195.58 119.38) (width 0.25) (layer F.Cu) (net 3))
 (segment (start 195.58 114.3) (end 193.04 114.3) (width 0.25) (layer F.Cu) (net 3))
 (segment (start 195.58 119.38) (end 195.58 114.3) (width 0.25) (layer F.Cu) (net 3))
 (segment (start 176.53 114.3) (end 185.42 114.3) (width 0.25) (layer F.Cu) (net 4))
 (segment (start 186.69 115.57) (end 193.04 115.57) (width 0.25) (layer F.Cu) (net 4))
 (segment (start 185.42 114.3) (end 186.69 115.57) (width 0.25) (layer F.Cu) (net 4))
 (segment (start 156.21 121.92) (end 163.83 121.92) (width 0.25) (layer F.Cu) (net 17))
 (segment (start 163.83 121.92) (end 166.37 124.46) (width 0.25) (layer F.Cu) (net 17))
 (segment (start 156.21 119.38) (end 166.37 119.38) (width 0.25) (layer F.Cu) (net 18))
 (segment (start 156.21 116.84) (end 163.83 116.84) (width 0.25) (layer F.Cu) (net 19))
 (segment (start 163.83 116.84) (end 166.37 114.3) (width 0.25) (layer F.Cu) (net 19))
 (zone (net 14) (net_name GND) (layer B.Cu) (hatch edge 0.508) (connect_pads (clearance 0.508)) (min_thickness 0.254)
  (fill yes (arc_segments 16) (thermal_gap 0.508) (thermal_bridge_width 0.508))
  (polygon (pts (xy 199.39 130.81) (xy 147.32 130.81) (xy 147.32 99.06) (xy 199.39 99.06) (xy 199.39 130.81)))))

